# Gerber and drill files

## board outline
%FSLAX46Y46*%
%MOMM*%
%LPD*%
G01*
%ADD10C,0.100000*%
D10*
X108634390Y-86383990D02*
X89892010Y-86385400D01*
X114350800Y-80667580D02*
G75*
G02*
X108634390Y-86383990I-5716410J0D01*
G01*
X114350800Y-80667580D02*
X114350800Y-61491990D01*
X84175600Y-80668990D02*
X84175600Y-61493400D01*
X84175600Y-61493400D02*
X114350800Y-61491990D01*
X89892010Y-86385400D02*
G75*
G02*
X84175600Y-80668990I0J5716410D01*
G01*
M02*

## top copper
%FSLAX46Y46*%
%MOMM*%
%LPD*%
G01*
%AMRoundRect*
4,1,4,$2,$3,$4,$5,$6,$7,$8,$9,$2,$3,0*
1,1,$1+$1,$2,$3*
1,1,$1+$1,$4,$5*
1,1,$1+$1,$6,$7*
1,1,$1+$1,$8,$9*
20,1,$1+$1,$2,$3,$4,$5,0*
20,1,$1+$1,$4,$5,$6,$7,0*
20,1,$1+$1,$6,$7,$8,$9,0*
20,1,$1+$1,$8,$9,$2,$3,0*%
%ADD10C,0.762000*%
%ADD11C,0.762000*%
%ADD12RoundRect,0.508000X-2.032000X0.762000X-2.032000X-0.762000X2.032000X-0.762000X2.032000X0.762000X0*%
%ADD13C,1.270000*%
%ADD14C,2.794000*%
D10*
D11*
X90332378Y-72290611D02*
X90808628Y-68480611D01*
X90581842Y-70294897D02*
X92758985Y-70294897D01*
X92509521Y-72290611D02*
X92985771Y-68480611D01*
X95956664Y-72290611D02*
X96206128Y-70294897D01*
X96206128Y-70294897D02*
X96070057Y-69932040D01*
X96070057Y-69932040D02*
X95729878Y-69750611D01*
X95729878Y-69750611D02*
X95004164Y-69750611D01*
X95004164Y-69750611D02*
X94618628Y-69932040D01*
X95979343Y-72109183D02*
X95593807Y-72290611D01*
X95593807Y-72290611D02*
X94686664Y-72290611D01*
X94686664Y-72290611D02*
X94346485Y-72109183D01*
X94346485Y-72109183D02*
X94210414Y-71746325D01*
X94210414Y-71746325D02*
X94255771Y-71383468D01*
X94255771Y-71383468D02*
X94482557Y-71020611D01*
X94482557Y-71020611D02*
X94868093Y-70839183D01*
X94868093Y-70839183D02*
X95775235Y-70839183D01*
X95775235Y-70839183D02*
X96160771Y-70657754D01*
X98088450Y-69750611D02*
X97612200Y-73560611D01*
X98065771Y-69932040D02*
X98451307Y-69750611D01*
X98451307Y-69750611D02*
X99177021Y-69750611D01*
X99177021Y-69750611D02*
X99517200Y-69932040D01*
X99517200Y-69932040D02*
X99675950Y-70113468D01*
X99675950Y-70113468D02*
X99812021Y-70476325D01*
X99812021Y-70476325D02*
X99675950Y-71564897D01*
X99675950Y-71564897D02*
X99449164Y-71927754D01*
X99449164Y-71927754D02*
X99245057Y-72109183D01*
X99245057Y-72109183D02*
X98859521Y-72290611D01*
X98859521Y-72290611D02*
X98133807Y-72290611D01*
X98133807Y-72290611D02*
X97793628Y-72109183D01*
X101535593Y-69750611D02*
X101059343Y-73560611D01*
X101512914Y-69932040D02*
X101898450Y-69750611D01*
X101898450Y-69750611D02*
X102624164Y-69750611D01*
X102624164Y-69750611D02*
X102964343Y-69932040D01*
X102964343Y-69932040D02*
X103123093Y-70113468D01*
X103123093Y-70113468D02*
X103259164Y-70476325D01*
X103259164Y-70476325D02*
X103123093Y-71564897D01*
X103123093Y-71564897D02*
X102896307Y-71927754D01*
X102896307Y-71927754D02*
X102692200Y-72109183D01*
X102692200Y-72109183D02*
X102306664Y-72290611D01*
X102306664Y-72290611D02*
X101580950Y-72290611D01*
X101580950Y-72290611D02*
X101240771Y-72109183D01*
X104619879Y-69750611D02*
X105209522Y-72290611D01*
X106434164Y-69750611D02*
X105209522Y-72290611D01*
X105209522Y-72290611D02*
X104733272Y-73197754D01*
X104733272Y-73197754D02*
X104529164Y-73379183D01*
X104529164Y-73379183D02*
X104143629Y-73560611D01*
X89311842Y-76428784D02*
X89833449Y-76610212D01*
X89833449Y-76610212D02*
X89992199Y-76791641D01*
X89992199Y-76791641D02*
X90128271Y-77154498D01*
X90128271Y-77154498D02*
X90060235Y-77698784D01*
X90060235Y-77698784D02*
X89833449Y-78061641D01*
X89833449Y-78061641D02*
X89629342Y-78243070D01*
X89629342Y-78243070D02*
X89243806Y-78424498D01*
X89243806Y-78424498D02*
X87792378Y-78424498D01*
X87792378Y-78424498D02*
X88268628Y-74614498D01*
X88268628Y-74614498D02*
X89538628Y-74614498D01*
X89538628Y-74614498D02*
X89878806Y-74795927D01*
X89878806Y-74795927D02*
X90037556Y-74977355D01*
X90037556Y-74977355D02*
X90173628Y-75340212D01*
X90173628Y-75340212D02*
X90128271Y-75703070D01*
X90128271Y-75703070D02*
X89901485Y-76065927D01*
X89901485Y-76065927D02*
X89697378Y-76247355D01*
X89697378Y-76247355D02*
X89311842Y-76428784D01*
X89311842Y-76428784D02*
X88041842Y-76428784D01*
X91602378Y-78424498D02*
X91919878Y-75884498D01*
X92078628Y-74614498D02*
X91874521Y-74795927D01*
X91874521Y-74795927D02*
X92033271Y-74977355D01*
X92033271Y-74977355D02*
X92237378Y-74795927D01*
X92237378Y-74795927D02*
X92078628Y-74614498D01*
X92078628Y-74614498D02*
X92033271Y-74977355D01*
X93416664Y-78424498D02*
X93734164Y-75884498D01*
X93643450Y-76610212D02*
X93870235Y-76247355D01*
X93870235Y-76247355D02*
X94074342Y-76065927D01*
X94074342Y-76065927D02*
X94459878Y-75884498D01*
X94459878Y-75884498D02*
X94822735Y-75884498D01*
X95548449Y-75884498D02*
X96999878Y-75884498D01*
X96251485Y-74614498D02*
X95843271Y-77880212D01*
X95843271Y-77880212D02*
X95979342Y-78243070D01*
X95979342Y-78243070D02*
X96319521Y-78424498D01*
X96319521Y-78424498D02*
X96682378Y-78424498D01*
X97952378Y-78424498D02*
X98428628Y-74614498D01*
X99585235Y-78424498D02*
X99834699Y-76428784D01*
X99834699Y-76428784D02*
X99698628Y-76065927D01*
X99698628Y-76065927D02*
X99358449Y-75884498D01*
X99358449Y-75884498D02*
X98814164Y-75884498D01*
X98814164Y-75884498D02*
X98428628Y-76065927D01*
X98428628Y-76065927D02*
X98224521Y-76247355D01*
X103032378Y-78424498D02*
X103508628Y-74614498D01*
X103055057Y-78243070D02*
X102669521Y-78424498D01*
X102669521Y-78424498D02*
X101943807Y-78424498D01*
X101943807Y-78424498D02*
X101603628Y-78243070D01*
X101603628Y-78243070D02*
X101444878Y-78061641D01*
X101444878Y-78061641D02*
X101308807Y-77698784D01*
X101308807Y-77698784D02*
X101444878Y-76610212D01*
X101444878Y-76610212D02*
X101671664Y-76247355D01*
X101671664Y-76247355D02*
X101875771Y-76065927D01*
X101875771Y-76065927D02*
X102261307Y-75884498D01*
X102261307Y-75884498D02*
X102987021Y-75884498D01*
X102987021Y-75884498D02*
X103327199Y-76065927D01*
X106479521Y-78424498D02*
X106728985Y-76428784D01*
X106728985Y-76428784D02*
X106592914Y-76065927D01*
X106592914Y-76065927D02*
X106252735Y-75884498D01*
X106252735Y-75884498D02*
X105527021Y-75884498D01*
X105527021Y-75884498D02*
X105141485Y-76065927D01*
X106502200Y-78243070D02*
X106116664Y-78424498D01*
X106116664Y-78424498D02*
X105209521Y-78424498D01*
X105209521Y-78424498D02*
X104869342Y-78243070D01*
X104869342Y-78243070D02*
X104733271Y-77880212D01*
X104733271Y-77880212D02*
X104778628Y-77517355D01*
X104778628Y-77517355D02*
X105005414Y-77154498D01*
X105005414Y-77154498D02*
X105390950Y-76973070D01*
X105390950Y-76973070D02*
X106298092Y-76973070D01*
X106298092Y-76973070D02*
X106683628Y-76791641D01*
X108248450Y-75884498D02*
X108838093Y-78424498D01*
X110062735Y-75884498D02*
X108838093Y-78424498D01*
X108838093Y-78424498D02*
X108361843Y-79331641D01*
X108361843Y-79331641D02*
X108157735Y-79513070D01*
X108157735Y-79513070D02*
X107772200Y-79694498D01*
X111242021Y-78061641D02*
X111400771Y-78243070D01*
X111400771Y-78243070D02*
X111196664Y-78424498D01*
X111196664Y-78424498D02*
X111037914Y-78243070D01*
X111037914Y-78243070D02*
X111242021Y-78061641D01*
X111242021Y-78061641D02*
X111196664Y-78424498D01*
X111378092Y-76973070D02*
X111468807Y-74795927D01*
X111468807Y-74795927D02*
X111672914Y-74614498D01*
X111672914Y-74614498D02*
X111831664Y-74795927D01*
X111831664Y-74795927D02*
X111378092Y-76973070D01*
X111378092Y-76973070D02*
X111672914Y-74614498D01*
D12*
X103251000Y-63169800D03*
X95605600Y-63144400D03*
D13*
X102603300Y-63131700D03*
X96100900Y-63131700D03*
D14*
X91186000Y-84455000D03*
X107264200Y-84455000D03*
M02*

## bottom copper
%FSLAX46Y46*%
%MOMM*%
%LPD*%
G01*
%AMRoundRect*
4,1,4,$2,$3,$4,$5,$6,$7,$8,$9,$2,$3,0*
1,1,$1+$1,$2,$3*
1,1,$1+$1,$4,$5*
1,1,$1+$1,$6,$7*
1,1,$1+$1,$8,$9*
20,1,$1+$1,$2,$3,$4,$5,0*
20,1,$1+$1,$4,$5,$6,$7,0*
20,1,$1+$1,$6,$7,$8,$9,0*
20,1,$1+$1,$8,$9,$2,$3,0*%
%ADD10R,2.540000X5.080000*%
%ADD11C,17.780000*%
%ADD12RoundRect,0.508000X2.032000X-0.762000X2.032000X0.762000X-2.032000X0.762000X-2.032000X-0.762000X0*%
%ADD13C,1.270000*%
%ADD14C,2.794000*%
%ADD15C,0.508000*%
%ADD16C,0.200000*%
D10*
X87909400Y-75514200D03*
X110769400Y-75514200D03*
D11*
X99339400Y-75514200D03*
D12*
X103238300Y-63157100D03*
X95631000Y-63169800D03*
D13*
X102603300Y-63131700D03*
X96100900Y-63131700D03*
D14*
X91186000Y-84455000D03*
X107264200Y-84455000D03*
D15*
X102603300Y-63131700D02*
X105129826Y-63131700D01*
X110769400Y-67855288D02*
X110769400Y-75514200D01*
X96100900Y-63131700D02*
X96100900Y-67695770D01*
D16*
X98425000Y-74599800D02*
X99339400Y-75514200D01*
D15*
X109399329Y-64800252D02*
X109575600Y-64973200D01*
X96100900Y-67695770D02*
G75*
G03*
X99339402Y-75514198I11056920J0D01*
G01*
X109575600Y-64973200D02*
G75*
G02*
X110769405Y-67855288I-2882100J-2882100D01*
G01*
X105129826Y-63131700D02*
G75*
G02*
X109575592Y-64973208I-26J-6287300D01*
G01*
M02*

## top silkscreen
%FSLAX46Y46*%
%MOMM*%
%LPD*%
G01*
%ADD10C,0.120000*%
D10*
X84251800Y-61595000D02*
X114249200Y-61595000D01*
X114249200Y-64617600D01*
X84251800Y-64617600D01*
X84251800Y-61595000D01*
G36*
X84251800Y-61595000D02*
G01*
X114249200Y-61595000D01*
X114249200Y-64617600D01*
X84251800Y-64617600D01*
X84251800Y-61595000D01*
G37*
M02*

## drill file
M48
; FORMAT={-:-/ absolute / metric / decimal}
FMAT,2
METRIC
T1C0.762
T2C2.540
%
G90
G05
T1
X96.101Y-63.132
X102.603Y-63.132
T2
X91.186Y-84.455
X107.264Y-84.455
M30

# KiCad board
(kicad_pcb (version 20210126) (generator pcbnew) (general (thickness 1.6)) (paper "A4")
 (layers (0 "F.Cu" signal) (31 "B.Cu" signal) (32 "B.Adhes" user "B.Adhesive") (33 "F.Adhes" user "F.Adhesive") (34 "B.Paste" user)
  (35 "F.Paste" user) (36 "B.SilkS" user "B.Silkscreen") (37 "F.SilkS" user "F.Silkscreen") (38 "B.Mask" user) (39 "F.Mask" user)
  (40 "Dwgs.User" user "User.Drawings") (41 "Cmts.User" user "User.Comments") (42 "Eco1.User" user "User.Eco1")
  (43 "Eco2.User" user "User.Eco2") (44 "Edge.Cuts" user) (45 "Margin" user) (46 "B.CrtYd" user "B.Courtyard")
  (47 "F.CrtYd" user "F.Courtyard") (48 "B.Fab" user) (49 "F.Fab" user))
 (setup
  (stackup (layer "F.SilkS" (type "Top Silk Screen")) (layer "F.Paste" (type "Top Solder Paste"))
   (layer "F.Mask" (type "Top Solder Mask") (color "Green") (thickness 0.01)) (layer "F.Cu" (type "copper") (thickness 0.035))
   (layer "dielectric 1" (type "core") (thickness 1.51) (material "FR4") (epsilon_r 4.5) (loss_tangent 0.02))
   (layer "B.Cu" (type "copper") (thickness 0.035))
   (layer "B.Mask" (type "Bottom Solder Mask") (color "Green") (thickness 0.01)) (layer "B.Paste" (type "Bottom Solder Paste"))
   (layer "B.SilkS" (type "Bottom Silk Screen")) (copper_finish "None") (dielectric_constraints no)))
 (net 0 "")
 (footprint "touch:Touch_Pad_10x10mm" (layer "F.Cu") (at 102.3366 63.5762 -90)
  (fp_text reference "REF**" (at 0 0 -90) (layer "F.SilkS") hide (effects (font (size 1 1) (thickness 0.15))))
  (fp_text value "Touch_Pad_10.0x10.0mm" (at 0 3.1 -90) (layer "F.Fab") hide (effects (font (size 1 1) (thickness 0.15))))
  (pad "1" smd roundrect (at -0.4064 -0.9144 270) (size 2.54 5.08) (layers "F.Cu" "F.Mask") (roundrect_rratio 0.2)))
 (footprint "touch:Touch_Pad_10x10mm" (layer "F.Cu") (at 95.1865 63.5127 -90)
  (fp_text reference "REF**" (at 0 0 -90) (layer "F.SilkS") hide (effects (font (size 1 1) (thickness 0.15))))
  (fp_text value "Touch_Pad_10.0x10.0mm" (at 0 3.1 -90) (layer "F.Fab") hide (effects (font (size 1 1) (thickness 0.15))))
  (pad "1" smd roundrect (at -0.3683 -0.4191 270) (size 2.54 5.08) (layers "F.Cu" "F.Mask") (roundrect_rratio 0.2)))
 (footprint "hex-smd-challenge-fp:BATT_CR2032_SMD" (layer "B.Cu") (at 99.3394 75.5142 180)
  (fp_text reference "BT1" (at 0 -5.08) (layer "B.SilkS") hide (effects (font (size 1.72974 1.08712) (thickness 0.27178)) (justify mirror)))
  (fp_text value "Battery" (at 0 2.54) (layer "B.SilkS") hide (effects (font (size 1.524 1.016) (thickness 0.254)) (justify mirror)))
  (pad "1" smd rect (at 11.43 0 180) (locked) (size 2.54 5.08) (layers "B.Cu" "B.Paste" "B.Mask"))
  (pad "1" smd rect (at -11.43 0 180) (locked) (size 2.54 5.08) (layers "B.Cu" "B.Paste" "B.Mask"))
  (pad "2" smd circle (at 0 0 180) (locked) (size 17.78 17.78) (layers "B.Cu" "B.Paste" "B.Mask")))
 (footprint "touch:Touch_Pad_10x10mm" (layer "B.Cu") (at 101.7778 62.7888 90)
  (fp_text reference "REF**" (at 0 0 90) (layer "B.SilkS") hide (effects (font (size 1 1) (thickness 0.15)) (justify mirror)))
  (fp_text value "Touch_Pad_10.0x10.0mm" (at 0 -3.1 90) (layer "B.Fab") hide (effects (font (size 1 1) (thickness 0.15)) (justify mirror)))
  (pad "1" smd roundrect (at -0.3683 1.4605 90) (size 2.54 5.08) (layers "B.Cu" "B.Mask") (roundrect_rratio 0.2)))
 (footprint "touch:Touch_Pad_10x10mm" (layer "B.Cu") (at 95.1865 62.8523 90)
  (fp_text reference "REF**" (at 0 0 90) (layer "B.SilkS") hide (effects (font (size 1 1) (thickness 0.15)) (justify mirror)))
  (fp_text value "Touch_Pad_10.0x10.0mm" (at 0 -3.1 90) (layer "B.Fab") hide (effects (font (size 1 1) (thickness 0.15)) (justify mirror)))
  (pad "1" smd roundrect (at -0.3175 0.4445 90) (size 2.54 5.08) (layers "B.Cu" "B.Mask") (roundrect_rratio 0.2)))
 (gr_rect (start 84.2518 64.6176) (end 114.2492 61.595) (layer "F.SilkS") (width 0.12) (fill solid))
 (gr_line (start 108.63439 86.38399) (end 89.89201 86.3854) (layer "Edge.Cuts") (width 0.1))
 (gr_arc (start 108.63439 80.66758) (end 114.3508 80.66758) (angle 90) (layer "Edge.Cuts") (width 0.1))
 (gr_line (start 114.3508 80.66758) (end 114.3508 61.49199) (layer "Edge.Cuts") (width 0.1))
 (gr_line (start 84.1756 80.66899) (end 84.1756 61.4934) (layer "Edge.Cuts") (width 0.1))
 (gr_line (start 84.1756 61.4934) (end 114.3508 61.49199) (layer "Edge.Cuts") (width 0.1))
 (gr_arc (start 89.89201 80.66899) (end 84.1756 80.66899) (angle -90) (layer "Edge.Cuts") (width 0.1))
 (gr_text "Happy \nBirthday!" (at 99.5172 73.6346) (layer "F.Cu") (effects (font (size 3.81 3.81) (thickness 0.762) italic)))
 (via (at 102.6033 63.1317) (size 1.27) (drill 0.762) (layers "F.Cu" "B.Cu") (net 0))
 (via (at 96.1009 63.1317) (size 1.27) (drill 0.762) (layers "F.Cu" "B.Cu") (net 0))
 (via (at 91.186 84.455) (size 2.794) (drill 2.54) (layers "F.Cu" "B.Cu") (free) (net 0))
 (via (at 107.2642 84.455) (size 2.794) (drill 2.54) (layers "F.Cu" "B.Cu") (free) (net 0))
 (segment (start 102.6033 63.1317) (end 105.129826 63.1317) (width 0.508) (layer "B.Cu") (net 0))
 (segment (start 110.7694 67.855288) (end 110.7694 75.5142) (width 0.508) (layer "B.Cu") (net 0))
 (segment (start 96.1009 63.1317) (end 96.1009 67.69577) (width 0.508) (layer "B.Cu") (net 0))
 (segment (start 98.425 74.5998) (end 99.3394 75.5142) (width 0.2) (layer "B.Cu") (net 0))
 (segment (start 109.399329 64.800252) (end 109.5756 64.9732) (width 0.508) (layer "B.Cu") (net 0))
 (arc (start 96.1009 67.69577) (mid 96.942558 71.927073) (end 99.3394 75.5142) (width 0.508) (layer "B.Cu") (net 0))
 (arc (start 109.5756 64.9732) (mid 110.459141 66.295512) (end 110.7694 67.855288) (width 0.508) (layer "B.Cu") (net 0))
 (arc (start 105.129826 63.1317) (mid 107.535861 63.61029) (end 109.5756 64.9732) (width 0.508) (layer "B.Cu") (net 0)))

